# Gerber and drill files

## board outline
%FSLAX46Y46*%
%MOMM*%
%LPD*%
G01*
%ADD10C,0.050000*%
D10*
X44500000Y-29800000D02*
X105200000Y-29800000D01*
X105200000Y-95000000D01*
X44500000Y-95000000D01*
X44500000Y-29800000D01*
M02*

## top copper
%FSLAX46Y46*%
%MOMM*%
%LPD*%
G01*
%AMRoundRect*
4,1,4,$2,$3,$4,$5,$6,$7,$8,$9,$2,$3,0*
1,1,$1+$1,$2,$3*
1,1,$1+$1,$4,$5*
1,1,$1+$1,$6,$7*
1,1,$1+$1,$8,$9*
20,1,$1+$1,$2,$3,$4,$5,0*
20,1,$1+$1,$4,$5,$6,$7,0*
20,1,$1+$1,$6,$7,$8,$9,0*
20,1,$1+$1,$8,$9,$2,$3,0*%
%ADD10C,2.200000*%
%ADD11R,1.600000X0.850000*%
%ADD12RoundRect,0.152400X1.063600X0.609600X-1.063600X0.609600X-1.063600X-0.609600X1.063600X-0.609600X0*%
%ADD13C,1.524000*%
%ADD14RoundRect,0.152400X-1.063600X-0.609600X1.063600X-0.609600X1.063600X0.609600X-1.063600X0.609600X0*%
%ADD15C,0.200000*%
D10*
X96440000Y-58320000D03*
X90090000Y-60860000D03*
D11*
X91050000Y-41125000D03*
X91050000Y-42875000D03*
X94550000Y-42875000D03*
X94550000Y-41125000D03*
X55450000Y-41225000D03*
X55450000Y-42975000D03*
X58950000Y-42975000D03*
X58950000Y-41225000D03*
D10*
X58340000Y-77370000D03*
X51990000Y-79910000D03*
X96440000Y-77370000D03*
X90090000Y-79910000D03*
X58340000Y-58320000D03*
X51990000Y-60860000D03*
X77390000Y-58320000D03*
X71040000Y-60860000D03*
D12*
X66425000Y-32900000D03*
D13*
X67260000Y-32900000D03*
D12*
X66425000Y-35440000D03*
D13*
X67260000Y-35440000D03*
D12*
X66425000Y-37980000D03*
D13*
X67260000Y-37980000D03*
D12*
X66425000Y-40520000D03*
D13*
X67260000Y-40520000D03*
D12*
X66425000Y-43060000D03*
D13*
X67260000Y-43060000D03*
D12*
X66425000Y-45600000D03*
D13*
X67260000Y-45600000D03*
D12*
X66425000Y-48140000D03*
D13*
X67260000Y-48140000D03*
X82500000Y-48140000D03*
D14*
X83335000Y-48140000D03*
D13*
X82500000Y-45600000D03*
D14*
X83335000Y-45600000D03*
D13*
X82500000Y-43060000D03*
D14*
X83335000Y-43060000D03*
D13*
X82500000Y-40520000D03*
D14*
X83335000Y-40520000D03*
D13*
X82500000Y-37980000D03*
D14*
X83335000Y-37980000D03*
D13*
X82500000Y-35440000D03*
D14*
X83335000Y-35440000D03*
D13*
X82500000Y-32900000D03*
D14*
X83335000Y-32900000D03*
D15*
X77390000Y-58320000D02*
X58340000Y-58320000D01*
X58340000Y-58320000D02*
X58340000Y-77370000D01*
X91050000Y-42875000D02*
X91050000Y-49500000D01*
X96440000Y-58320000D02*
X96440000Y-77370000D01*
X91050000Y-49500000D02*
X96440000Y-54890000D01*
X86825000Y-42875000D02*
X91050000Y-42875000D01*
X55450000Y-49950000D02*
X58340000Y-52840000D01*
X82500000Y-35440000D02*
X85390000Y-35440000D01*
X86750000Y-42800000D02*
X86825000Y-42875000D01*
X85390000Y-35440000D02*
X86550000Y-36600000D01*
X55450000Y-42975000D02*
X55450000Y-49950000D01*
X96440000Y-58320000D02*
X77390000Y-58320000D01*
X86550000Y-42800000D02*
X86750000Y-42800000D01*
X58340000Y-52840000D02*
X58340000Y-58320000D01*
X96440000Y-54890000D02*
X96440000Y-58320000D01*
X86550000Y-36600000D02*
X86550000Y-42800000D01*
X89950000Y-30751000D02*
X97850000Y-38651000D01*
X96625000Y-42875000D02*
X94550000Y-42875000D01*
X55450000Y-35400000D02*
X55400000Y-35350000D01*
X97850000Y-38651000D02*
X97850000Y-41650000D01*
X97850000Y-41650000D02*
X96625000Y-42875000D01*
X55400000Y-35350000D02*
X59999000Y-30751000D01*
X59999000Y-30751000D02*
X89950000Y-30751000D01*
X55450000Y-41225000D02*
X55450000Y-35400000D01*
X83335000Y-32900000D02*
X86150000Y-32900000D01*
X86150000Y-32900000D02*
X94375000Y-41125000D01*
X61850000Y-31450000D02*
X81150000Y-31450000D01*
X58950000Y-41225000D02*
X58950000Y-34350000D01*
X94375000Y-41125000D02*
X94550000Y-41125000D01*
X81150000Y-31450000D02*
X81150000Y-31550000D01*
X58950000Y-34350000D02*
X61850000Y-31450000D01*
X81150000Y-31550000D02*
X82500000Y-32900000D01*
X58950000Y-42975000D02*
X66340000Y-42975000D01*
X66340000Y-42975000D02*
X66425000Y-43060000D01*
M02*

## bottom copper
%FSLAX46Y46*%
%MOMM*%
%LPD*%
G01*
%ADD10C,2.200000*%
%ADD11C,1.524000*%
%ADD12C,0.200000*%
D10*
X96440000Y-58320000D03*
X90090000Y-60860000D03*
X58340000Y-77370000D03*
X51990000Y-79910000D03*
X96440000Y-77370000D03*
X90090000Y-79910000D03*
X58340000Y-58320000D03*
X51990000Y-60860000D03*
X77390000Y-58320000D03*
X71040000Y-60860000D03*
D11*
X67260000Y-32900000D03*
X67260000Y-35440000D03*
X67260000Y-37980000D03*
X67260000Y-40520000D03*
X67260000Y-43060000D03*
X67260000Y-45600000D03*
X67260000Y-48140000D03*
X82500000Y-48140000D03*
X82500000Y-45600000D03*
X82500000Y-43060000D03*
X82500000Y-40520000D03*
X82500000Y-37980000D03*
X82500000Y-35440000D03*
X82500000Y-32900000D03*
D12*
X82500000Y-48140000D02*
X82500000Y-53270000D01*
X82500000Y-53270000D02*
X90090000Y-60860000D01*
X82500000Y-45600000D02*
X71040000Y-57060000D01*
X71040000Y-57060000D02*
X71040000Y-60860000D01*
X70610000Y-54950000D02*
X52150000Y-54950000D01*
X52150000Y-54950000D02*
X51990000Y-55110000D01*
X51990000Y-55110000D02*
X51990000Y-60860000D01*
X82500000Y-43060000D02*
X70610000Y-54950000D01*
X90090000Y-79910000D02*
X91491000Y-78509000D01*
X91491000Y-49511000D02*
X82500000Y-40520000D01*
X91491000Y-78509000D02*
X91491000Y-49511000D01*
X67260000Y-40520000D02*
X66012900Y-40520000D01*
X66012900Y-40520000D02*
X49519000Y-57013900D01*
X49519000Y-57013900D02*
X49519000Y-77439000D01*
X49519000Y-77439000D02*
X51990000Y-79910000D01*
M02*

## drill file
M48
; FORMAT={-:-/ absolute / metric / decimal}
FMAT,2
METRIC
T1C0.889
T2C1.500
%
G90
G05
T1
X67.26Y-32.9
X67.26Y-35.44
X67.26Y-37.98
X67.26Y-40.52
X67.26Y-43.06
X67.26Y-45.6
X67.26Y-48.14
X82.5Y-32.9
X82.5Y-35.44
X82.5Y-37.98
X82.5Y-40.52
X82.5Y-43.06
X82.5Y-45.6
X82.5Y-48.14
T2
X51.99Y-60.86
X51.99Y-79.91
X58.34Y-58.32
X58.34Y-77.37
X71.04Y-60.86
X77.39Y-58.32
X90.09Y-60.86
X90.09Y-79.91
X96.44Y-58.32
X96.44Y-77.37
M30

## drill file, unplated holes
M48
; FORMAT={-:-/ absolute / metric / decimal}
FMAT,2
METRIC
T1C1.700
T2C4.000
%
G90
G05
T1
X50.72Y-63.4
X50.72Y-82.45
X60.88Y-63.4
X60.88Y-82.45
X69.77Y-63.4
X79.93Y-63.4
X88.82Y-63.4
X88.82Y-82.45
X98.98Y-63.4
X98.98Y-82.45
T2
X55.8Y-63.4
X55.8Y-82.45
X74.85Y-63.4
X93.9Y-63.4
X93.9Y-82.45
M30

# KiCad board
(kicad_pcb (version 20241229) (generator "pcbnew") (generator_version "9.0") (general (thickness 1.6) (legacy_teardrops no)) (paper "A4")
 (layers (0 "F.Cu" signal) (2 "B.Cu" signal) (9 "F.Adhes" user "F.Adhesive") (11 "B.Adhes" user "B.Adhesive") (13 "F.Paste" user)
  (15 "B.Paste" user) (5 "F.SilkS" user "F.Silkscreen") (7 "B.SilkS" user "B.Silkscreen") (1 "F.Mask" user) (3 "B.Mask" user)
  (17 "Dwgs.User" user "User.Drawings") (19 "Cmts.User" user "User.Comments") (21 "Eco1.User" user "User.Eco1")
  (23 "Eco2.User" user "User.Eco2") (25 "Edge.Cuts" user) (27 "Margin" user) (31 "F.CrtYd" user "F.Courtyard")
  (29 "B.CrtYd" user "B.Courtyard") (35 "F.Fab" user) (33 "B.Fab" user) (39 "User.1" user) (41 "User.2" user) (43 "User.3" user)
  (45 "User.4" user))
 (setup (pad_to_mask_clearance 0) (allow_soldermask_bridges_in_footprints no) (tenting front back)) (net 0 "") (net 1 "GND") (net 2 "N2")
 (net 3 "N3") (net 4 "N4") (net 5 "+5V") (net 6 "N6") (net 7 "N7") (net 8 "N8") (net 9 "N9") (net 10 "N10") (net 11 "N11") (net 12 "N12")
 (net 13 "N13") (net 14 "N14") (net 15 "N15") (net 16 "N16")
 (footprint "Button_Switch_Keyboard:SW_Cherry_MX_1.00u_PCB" (layer "F.Cu") (at 96.44 58.32)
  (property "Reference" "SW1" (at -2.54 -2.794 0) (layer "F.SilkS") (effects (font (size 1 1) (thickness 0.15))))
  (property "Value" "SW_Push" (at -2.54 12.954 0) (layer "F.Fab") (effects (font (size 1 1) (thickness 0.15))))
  (pad "" np_thru_hole circle (at -7.62 5.08) (size 1.7 1.7) (drill 1.7) (layers "*.Cu" "*.Mask"))
  (pad "" np_thru_hole circle (at -2.54 5.08) (size 4 4) (drill 4) (layers "*.Cu" "*.Mask"))
  (pad "" np_thru_hole circle (at 2.54 5.08) (size 1.7 1.7) (drill 1.7) (layers "*.Cu" "*.Mask"))
  (pad "1" thru_hole circle (at 0 0) (size 2.2 2.2) (drill 1.5) (layers "*.Cu" "*.Mask") (remove_unused_layers no) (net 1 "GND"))
  (pad "2" thru_hole circle (at -6.35 2.54) (size 2.2 2.2) (drill 1.5) (layers "*.Cu" "*.Mask") (remove_unused_layers no) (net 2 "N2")))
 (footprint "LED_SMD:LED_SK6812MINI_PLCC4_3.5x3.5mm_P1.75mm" (layer "F.Cu") (at 92.8 42)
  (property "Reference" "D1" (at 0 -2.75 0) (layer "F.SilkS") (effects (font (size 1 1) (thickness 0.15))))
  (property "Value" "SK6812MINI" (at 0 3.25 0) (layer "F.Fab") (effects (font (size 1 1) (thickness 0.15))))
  (pad "1" smd rect (at -1.75 -0.875) (size 1.6 0.85) (layers "F.Cu" "F.Mask" "F.Paste") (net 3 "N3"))
  (pad "2" smd rect (at -1.75 0.875) (size 1.6 0.85) (layers "F.Cu" "F.Mask" "F.Paste") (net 1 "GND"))
  (pad "3" smd rect (at 1.75 0.875) (size 1.6 0.85) (layers "F.Cu" "F.Mask" "F.Paste") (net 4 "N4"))
  (pad "4" smd rect (at 1.75 -0.875) (size 1.6 0.85) (layers "F.Cu" "F.Mask" "F.Paste") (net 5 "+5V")))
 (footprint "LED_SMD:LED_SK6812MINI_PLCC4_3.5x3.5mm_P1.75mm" (layer "F.Cu") (at 57.2 42.1)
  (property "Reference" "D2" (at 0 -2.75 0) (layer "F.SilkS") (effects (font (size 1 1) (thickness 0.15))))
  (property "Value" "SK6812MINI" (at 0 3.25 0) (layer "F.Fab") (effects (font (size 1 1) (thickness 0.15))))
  (pad "1" smd rect (at -1.75 -0.875) (size 1.6 0.85) (layers "F.Cu" "F.Mask" "F.Paste") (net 4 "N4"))
  (pad "2" smd rect (at -1.75 0.875) (size 1.6 0.85) (layers "F.Cu" "F.Mask" "F.Paste") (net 1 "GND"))
  (pad "3" smd rect (at 1.75 0.875) (size 1.6 0.85) (layers "F.Cu" "F.Mask" "F.Paste") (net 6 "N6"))
  (pad "4" smd rect (at 1.75 -0.875) (size 1.6 0.85) (layers "F.Cu" "F.Mask" "F.Paste") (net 5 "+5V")))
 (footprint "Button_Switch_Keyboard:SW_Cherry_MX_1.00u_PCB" (layer "F.Cu") (at 58.34 77.37)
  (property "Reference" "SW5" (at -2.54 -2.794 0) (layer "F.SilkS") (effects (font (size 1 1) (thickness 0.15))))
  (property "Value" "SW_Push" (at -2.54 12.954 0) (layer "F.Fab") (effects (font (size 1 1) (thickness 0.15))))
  (pad "" np_thru_hole circle (at -7.62 5.08) (size 1.7 1.7) (drill 1.7) (layers "*.Cu" "*.Mask"))
  (pad "" np_thru_hole circle (at -2.54 5.08) (size 4 4) (drill 4) (layers "*.Cu" "*.Mask"))
  (pad "" np_thru_hole circle (at 2.54 5.08) (size 1.7 1.7) (drill 1.7) (layers "*.Cu" "*.Mask"))
  (pad "1" thru_hole circle (at 0 0) (size 2.2 2.2) (drill 1.5) (layers "*.Cu" "*.Mask") (remove_unused_layers no) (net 1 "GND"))
  (pad "2" thru_hole circle (at -6.35 2.54) (size 2.2 2.2) (drill 1.5) (layers "*.Cu" "*.Mask") (remove_unused_layers no) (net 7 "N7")))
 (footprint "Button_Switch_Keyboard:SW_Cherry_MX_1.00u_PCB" (layer "F.Cu") (at 96.44 77.37)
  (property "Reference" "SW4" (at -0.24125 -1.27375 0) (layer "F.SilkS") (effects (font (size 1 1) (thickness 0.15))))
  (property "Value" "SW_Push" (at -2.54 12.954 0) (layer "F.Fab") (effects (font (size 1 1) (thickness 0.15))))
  (pad "" np_thru_hole circle (at -7.62 5.08) (size 1.7 1.7) (drill 1.7) (layers "*.Cu" "*.Mask"))
  (pad "" np_thru_hole circle (at -2.54 5.08) (size 4 4) (drill 4) (layers "*.Cu" "*.Mask"))
  (pad "" np_thru_hole circle (at 2.54 5.08) (size 1.7 1.7) (drill 1.7) (layers "*.Cu" "*.Mask"))
  (pad "1" thru_hole circle (at 0 0) (size 2.2 2.2) (drill 1.5) (layers "*.Cu" "*.Mask") (remove_unused_layers no) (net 1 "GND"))
  (pad "2" thru_hole circle (at -6.35 2.54) (size 2.2 2.2) (drill 1.5) (layers "*.Cu" "*.Mask") (remove_unused_layers no) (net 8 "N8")))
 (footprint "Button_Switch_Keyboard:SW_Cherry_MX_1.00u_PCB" (layer "F.Cu") (at 58.34 58.32)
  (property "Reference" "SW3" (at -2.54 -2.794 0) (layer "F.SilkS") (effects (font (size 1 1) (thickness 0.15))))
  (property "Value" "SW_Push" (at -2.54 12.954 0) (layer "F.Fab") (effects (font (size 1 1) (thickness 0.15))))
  (pad "" np_thru_hole circle (at -7.62 5.08) (size 1.7 1.7) (drill 1.7) (layers "*.Cu" "*.Mask"))
  (pad "" np_thru_hole circle (at -2.54 5.08) (size 4 4) (drill 4) (layers "*.Cu" "*.Mask"))
  (pad "" np_thru_hole circle (at 2.54 5.08) (size 1.7 1.7) (drill 1.7) (layers "*.Cu" "*.Mask"))
  (pad "1" thru_hole circle (at 0 0) (size 2.2 2.2) (drill 1.5) (layers "*.Cu" "*.Mask") (remove_unused_layers no) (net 1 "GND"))
  (pad "2" thru_hole circle (at -6.35 2.54) (size 2.2 2.2) (drill 1.5) (layers "*.Cu" "*.Mask") (remove_unused_layers no) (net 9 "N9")))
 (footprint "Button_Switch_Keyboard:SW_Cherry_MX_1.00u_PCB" (layer "F.Cu") (at 77.39 58.32)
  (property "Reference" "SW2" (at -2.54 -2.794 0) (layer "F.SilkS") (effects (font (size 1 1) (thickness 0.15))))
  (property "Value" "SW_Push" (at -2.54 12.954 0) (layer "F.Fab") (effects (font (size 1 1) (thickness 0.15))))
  (pad "" np_thru_hole circle (at -7.62 5.08) (size 1.7 1.7) (drill 1.7) (layers "*.Cu" "*.Mask"))
  (pad "" np_thru_hole circle (at -2.54 5.08) (size 4 4) (drill 4) (layers "*.Cu" "*.Mask"))
  (pad "" np_thru_hole circle (at 2.54 5.08) (size 1.7 1.7) (drill 1.7) (layers "*.Cu" "*.Mask"))
  (pad "1" thru_hole circle (at 0 0) (size 2.2 2.2) (drill 1.5) (layers "*.Cu" "*.Mask") (remove_unused_layers no) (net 1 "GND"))
  (pad "2" thru_hole circle (at -6.35 2.54) (size 2.2 2.2) (drill 1.5) (layers "*.Cu" "*.Mask") (remove_unused_layers no) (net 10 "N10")))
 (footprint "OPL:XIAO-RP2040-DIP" (layer "F.Cu") (at 74.88 40.52)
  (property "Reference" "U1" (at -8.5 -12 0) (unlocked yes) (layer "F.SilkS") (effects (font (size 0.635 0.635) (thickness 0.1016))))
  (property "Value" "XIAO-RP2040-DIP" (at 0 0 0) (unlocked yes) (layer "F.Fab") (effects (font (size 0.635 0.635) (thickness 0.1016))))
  (pad "1" smd roundrect (at -8.455 -7.62 180) (size 2.432 1.524) (layers "F.Cu" "F.Mask") (roundrect_rratio 0.1) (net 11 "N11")
   (thermal_bridge_angle 45))
  (pad "1" thru_hole circle (at -7.62 -7.62 180) (size 1.524 1.524) (drill 0.889) (layers "*.Cu" "*.Mask") (remove_unused_layers no)
   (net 11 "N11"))
  (pad "2" smd roundrect (at -8.455 -5.08 180) (size 2.432 1.524) (layers "F.Cu" "F.Mask") (roundrect_rratio 0.1) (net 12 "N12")
   (thermal_bridge_angle 45))
  (pad "2" thru_hole circle (at -7.62 -5.08 180) (size 1.524 1.524) (drill 0.889) (layers "*.Cu" "*.Mask") (remove_unused_layers no)
   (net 12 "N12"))
  (pad "3" smd roundrect (at -8.455 -2.54 180) (size 2.432 1.524) (layers "F.Cu" "F.Mask") (roundrect_rratio 0.1) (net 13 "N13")
   (thermal_bridge_angle 45))
  (pad "3" thru_hole circle (at -7.62 -2.54 180) (size 1.524 1.524) (drill 0.889) (layers "*.Cu" "*.Mask") (remove_unused_layers no)
   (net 13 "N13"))
  (pad "4" smd roundrect (at -8.455 0 180) (size 2.432 1.524) (layers "F.Cu" "F.Mask") (roundrect_rratio 0.1) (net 7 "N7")
   (thermal_bridge_angle 45))
  (pad "4" thru_hole circle (at -7.62 0 180) (size 1.524 1.524) (drill 0.889) (layers "*.Cu" "*.Mask") (remove_unused_layers no)
   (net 7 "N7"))
  (pad "5" smd roundrect (at -8.455 2.54 180) (size 2.432 1.524) (layers "F.Cu" "F.Mask") (roundrect_rratio 0.1) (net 6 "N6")
   (thermal_bridge_angle 45))
  (pad "5" thru_hole circle (at -7.62 2.54 180) (size 1.524 1.524) (drill 0.889) (layers "*.Cu" "*.Mask") (remove_unused_layers no)
   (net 6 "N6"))
  (pad "6" smd roundrect (at -8.455 5.08 180) (size 2.432 1.524) (layers "F.Cu" "F.Mask") (roundrect_rratio 0.1) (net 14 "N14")
   (thermal_bridge_angle 45))
  (pad "6" thru_hole circle (at -7.62 5.08 180) (size 1.524 1.524) (drill 0.889) (layers "*.Cu" "*.Mask") (remove_unused_layers no)
   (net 14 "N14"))
  (pad "7" smd roundrect (at -8.455 7.62 180) (size 2.432 1.524) (layers "F.Cu" "F.Mask") (roundrect_rratio 0.1) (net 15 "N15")
   (thermal_bridge_angle 45))
  (pad "7" thru_hole circle (at -7.62 7.62 180) (size 1.524 1.524) (drill 0.889) (layers "*.Cu" "*.Mask") (remove_unused_layers no)
   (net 15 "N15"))
  (pad "8" thru_hole circle (at 7.62 7.62) (size 1.524 1.524) (drill 0.889) (layers "*.Cu" "*.Mask") (remove_unused_layers no) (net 2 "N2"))
  (pad "8" smd roundrect (at 8.455 7.62) (size 2.432 1.524) (layers "F.Cu" "F.Mask") (roundrect_rratio 0.1) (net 2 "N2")
   (thermal_bridge_angle 45))
  (pad "9" thru_hole circle (at 7.62 5.08) (size 1.524 1.524) (drill 0.889) (layers "*.Cu" "*.Mask") (remove_unused_layers no)
   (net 10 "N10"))
  (pad "9" smd roundrect (at 8.455 5.08) (size 2.432 1.524) (layers "F.Cu" "F.Mask") (roundrect_rratio 0.1) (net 10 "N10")
   (thermal_bridge_angle 45))
  (pad "10" thru_hole circle (at 7.62 2.54) (size 1.524 1.524) (drill 0.889) (layers "*.Cu" "*.Mask") (remove_unused_layers no) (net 9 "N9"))
  (pad "10" smd roundrect (at 8.455 2.54) (size 2.432 1.524) (layers "F.Cu" "F.Mask") (roundrect_rratio 0.1) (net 9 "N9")
   (thermal_bridge_angle 45))
  (pad "11" thru_hole circle (at 7.62 0) (size 1.524 1.524) (drill 0.889) (layers "*.Cu" "*.Mask") (remove_unused_layers no) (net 8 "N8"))
  (pad "11" smd roundrect (at 8.455 0) (size 2.432 1.524) (layers "F.Cu" "F.Mask") (roundrect_rratio 0.1) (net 8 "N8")
   (thermal_bridge_angle 45))
  (pad "12" thru_hole circle (at 7.62 -2.54) (size 1.524 1.524) (drill 0.889) (layers "*.Cu" "*.Mask") (remove_unused_layers no)
   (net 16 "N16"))
  (pad "12" smd roundrect (at 8.455 -2.54) (size 2.432 1.524) (layers "F.Cu" "F.Mask") (roundrect_rratio 0.1) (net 16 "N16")
   (thermal_bridge_angle 45))
  (pad "13" thru_hole circle (at 7.62 -5.08) (size 1.524 1.524) (drill 0.889) (layers "*.Cu" "*.Mask") (remove_unused_layers no)
   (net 1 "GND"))
  (pad "13" smd roundrect (at 8.455 -5.08) (size 2.432 1.524) (layers "F.Cu" "F.Mask") (roundrect_rratio 0.1) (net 1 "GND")
   (thermal_bridge_angle 45))
  (pad "14" thru_hole circle (at 7.62 -7.62) (size 1.524 1.524) (drill 0.889) (layers "*.Cu" "*.Mask") (remove_unused_layers no)
   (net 5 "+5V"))
  (pad "14" smd roundrect (at 8.455 -7.62) (size 2.432 1.524) (layers "F.Cu" "F.Mask") (roundrect_rratio 0.1) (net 5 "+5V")
   (thermal_bridge_angle 45)))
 (gr_rect (start 44.5 29.8) (end 105.2 95) (stroke (width 0.05) (type default)) (fill no) (layer "Edge.Cuts"))
 (segment (start 77.39 58.32) (end 58.34 58.32) (width 0.2) (layer "F.Cu") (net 1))
 (segment (start 58.34 58.32) (end 58.34 77.37) (width 0.2) (layer "F.Cu") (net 1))
 (segment (start 91.05 42.875) (end 91.05 49.5) (width 0.2) (layer "F.Cu") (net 1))
 (segment (start 96.44 58.32) (end 96.44 77.37) (width 0.2) (layer "F.Cu") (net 1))
 (segment (start 91.05 49.5) (end 96.44 54.89) (width 0.2) (layer "F.Cu") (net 1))
 (segment (start 86.825 42.875) (end 91.05 42.875) (width 0.2) (layer "F.Cu") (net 1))
 (segment (start 55.45 49.95) (end 58.34 52.84) (width 0.2) (layer "F.Cu") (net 1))
 (segment (start 82.5 35.44) (end 85.39 35.44) (width 0.2) (layer "F.Cu") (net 1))
 (segment (start 86.75 42.8) (end 86.825 42.875) (width 0.2) (layer "F.Cu") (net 1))
 (segment (start 85.39 35.44) (end 86.55 36.6) (width 0.2) (layer "F.Cu") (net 1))
 (segment (start 55.45 42.975) (end 55.45 49.95) (width 0.2) (layer "F.Cu") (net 1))
 (segment (start 96.44 58.32) (end 77.39 58.32) (width 0.2) (layer "F.Cu") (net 1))
 (segment (start 86.55 42.8) (end 86.75 42.8) (width 0.2) (layer "F.Cu") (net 1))
 (segment (start 58.34 52.84) (end 58.34 58.32) (width 0.2) (layer "F.Cu") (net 1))
 (segment (start 96.44 54.89) (end 96.44 58.32) (width 0.2) (layer "F.Cu") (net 1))
 (segment (start 86.55 36.6) (end 86.55 42.8) (width 0.2) (layer "F.Cu") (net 1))
 (segment (start 89.95 30.751) (end 97.85 38.651) (width 0.2) (layer "F.Cu") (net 4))
 (segment (start 96.625 42.875) (end 94.55 42.875) (width 0.2) (layer "F.Cu") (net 4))
 (segment (start 55.45 35.4) (end 55.4 35.35) (width 0.2) (layer "F.Cu") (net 4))
 (segment (start 97.85 38.651) (end 97.85 41.65) (width 0.2) (layer "F.Cu") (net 4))
 (segment (start 97.85 41.65) (end 96.625 42.875) (width 0.2) (layer "F.Cu") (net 4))
 (segment (start 55.4 35.35) (end 59.999 30.751) (width 0.2) (layer "F.Cu") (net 4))
 (segment (start 59.999 30.751) (end 89.95 30.751) (width 0.2) (layer "F.Cu") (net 4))
 (segment (start 55.45 41.225) (end 55.45 35.4) (width 0.2) (layer "F.Cu") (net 4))
 (segment (start 83.335 32.9) (end 86.15 32.9) (width 0.2) (layer "F.Cu") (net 5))
 (segment (start 86.15 32.9) (end 94.375 41.125) (width 0.2) (layer "F.Cu") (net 5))
 (segment (start 61.85 31.45) (end 81.15 31.45) (width 0.2) (layer "F.Cu") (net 5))
 (segment (start 58.95 41.225) (end 58.95 34.35) (width 0.2) (layer "F.Cu") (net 5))
 (segment (start 94.375 41.125) (end 94.55 41.125) (width 0.2) (layer "F.Cu") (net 5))
 (segment (start 81.15 31.45) (end 81.15 31.55) (width 0.2) (layer "F.Cu") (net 5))
 (segment (start 58.95 34.35) (end 61.85 31.45) (width 0.2) (layer "F.Cu") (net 5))
 (segment (start 81.15 31.55) (end 82.5 32.9) (width 0.2) (layer "F.Cu") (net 5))
 (segment (start 58.95 42.975) (end 66.34 42.975) (width 0.2) (layer "F.Cu") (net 6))
 (segment (start 66.34 42.975) (end 66.425 43.06) (width 0.2) (layer "F.Cu") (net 6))
 (segment (start 82.5 48.14) (end 82.5 53.27) (width 0.2) (layer "B.Cu") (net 2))
 (segment (start 82.5 53.27) (end 90.09 60.86) (width 0.2) (layer "B.Cu") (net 2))
 (segment (start 82.5 45.6) (end 71.04 57.06) (width 0.2) (layer "B.Cu") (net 10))
 (segment (start 71.04 57.06) (end 71.04 60.86) (width 0.2) (layer "B.Cu") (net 10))
 (segment (start 70.61 54.95) (end 52.15 54.95) (width 0.2) (layer "B.Cu") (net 9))
 (segment (start 52.15 54.95) (end 51.99 55.11) (width 0.2) (layer "B.Cu") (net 9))
 (segment (start 51.99 55.11) (end 51.99 60.86) (width 0.2) (layer "B.Cu") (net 9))
 (segment (start 82.5 43.06) (end 70.61 54.95) (width 0.2) (layer "B.Cu") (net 9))
 (segment (start 90.09 79.91) (end 91.491 78.509) (width 0.2) (layer "B.Cu") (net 8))
 (segment (start 91.491 49.511) (end 82.5 40.52) (width 0.2) (layer "B.Cu") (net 8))
 (segment (start 91.491 78.509) (end 91.491 49.511) (width 0.2) (layer "B.Cu") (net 8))
 (segment (start 67.26 40.52) (end 66.0129 40.52) (width 0.2) (layer "B.Cu") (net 7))
 (segment (start 66.0129 40.52) (end 49.519 57.0139) (width 0.2) (layer "B.Cu") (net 7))
 (segment (start 49.519 57.0139) (end 49.519 77.439) (width 0.2) (layer "B.Cu") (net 7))
 (segment (start 49.519 77.439) (end 51.99 79.91) (width 0.2) (layer "B.Cu") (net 7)))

